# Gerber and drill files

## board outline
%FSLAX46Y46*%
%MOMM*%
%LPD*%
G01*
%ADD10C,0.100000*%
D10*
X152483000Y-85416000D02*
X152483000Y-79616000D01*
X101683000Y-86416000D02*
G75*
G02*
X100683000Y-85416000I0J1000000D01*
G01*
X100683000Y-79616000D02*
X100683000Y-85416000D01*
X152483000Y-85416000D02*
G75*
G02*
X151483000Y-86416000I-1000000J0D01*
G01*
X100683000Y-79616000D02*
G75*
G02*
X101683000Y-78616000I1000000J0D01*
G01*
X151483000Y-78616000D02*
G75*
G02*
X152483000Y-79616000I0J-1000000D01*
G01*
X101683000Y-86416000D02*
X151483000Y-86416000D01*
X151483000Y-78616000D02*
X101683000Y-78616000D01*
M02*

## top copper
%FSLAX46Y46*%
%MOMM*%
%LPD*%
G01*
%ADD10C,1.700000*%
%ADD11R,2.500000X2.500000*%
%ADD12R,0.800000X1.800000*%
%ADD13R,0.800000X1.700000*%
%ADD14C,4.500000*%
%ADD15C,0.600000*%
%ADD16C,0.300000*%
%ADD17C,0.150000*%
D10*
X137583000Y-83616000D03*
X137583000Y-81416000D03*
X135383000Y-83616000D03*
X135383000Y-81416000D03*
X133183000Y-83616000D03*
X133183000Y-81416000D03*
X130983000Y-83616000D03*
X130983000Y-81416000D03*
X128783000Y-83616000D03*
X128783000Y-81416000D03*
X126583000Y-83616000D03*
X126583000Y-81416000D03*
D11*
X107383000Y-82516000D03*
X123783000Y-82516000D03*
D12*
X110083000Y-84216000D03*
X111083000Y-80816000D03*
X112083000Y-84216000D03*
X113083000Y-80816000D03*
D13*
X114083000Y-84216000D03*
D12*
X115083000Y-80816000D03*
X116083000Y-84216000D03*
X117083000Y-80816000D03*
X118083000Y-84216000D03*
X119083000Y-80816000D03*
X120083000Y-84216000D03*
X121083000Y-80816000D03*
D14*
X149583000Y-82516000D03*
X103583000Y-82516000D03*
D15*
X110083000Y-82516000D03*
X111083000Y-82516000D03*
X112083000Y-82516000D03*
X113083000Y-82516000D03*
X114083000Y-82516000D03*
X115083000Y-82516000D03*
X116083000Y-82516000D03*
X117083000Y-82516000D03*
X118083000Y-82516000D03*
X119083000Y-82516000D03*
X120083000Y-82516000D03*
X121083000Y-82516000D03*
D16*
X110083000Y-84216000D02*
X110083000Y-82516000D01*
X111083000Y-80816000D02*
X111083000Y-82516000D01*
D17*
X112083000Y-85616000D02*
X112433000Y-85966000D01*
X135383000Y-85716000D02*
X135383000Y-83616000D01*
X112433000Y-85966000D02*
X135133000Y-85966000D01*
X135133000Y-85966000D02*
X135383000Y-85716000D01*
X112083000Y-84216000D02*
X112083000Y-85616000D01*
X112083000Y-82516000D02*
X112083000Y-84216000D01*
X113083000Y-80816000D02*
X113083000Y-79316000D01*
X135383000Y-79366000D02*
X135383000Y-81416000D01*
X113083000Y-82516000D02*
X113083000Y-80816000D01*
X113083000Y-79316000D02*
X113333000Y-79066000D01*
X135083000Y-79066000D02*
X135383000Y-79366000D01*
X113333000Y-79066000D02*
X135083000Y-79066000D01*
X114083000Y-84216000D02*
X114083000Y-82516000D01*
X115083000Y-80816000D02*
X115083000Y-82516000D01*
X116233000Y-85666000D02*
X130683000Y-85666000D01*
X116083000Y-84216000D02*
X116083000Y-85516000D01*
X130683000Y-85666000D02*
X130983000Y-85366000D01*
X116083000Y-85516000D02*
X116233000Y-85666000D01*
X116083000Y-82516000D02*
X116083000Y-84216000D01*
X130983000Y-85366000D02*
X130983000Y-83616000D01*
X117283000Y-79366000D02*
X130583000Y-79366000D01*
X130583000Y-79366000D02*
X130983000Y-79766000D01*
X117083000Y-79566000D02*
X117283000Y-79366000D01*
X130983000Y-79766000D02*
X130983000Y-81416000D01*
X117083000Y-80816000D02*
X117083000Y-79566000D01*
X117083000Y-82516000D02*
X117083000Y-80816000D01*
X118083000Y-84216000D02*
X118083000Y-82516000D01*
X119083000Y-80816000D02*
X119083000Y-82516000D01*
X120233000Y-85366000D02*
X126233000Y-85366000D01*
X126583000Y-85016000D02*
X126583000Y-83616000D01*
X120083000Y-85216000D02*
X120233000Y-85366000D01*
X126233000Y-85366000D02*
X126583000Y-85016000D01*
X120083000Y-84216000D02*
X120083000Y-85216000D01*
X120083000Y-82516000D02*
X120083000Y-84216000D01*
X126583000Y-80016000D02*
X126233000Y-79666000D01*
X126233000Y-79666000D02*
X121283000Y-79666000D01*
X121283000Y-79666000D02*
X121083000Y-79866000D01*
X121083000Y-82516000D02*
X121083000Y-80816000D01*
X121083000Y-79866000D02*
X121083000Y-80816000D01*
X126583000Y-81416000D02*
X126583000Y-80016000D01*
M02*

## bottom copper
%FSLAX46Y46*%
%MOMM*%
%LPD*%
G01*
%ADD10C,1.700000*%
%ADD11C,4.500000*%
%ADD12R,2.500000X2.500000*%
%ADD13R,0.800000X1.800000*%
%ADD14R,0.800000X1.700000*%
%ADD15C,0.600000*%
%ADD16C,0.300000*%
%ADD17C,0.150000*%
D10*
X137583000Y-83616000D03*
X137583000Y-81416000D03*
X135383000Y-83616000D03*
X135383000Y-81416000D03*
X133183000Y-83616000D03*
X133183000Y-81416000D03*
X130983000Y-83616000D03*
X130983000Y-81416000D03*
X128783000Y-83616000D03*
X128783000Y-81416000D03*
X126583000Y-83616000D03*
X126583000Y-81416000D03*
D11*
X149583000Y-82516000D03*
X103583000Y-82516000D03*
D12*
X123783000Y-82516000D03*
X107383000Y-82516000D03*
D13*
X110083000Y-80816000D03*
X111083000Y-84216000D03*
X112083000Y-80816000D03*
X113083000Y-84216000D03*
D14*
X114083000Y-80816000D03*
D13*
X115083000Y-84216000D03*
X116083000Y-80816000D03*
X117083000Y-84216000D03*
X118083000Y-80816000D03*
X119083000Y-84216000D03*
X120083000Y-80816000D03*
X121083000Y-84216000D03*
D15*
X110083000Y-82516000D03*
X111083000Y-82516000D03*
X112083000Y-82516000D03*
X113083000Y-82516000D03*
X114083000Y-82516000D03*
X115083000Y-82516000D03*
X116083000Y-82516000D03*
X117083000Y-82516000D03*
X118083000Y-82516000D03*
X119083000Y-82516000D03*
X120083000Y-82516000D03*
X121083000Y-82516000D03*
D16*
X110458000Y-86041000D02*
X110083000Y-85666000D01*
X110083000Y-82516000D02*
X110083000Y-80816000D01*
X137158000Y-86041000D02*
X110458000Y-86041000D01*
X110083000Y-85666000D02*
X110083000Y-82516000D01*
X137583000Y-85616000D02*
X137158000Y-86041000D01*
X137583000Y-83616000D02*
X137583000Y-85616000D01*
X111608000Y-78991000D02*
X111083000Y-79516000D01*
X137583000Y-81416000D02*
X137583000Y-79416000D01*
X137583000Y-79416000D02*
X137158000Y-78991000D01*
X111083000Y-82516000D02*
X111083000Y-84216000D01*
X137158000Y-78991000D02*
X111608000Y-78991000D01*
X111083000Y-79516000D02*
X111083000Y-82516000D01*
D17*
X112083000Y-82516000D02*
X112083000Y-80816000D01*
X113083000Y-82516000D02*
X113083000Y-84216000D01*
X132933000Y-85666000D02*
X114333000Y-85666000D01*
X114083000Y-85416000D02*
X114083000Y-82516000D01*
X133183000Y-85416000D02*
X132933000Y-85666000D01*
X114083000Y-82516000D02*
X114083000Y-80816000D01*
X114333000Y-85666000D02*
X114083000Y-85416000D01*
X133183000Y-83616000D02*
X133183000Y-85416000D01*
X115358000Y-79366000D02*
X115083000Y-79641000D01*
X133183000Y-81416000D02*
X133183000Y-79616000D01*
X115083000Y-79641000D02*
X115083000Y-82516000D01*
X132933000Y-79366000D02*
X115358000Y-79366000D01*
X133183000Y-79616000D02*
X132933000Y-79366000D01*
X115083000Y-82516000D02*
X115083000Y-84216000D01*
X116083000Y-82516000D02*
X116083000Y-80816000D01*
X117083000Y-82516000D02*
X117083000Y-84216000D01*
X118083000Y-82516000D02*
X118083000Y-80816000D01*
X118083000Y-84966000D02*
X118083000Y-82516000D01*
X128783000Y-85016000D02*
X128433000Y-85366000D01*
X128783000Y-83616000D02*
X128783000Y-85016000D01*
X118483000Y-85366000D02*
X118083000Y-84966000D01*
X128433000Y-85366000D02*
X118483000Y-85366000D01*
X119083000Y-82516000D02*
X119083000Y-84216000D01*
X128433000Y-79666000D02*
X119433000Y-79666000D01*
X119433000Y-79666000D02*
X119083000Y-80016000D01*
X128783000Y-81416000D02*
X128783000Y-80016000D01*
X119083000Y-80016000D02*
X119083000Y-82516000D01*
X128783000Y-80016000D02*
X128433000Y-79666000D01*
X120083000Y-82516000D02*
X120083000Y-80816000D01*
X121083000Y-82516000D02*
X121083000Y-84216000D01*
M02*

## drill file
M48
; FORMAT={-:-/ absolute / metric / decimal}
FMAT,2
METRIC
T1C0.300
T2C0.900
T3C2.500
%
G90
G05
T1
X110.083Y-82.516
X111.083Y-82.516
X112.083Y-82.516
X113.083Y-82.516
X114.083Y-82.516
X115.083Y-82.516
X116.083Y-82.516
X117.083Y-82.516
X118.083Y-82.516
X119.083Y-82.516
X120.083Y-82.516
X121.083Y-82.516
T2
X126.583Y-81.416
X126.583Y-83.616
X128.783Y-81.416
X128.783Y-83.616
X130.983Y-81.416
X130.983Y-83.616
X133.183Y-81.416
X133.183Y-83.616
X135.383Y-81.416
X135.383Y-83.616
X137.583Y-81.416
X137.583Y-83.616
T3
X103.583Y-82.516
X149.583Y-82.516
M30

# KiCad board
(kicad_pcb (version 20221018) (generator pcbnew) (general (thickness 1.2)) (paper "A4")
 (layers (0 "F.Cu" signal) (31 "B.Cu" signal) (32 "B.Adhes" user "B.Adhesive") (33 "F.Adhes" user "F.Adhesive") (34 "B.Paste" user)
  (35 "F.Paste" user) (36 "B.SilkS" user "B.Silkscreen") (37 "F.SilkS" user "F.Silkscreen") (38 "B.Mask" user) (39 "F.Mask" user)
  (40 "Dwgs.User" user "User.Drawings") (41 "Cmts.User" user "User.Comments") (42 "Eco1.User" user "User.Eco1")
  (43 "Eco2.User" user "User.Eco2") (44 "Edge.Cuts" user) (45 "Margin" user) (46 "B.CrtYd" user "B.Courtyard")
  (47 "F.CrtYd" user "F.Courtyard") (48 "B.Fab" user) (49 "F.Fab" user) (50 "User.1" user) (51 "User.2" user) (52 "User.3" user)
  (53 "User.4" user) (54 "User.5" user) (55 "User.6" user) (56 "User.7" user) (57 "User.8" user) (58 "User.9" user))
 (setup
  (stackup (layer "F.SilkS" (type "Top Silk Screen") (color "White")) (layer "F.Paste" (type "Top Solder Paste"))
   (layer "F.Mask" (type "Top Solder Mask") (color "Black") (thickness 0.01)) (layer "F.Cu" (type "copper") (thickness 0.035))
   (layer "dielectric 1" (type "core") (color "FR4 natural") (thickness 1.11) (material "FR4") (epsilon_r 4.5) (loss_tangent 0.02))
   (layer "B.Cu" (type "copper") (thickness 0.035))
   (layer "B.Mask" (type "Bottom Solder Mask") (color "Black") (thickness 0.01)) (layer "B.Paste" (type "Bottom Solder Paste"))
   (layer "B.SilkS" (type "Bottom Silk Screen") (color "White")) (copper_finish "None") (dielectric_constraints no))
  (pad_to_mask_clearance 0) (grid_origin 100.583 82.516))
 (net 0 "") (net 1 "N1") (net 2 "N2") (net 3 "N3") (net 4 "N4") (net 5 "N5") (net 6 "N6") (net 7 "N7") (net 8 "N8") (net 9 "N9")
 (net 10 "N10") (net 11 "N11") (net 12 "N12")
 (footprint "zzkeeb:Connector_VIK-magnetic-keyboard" (layer "F.Cu") (at 132.083 82.516 90)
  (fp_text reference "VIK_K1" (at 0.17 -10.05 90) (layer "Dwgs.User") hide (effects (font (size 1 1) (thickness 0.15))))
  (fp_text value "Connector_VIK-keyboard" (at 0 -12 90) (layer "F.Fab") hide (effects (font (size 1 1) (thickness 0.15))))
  (pad "1" thru_hole circle (at -1.1 5.5 270) (size 1.7 1.7) (drill 0.9) (layers "*.Cu" "*.Mask") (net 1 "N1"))
  (pad "2" thru_hole circle (at 1.1 5.5 270) (size 1.7 1.7) (drill 0.9) (layers "*.Cu" "*.Mask") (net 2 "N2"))
  (pad "3" thru_hole circle (at -1.1 3.3 270) (size 1.7 1.7) (drill 0.9) (layers "*.Cu" "*.Mask") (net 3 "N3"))
  (pad "4" thru_hole circle (at 1.1 3.3 270) (size 1.7 1.7) (drill 0.9) (layers "*.Cu" "*.Mask") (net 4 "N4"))
  (pad "5" thru_hole circle (at -1.1 1.1 270) (size 1.7 1.7) (drill 0.9) (layers "*.Cu" "*.Mask") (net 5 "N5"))
  (pad "6" thru_hole circle (at 1.1 1.1 270) (size 1.7 1.7) (drill 0.9) (layers "*.Cu" "*.Mask") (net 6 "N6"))
  (pad "7" thru_hole circle (at -1.1 -1.1 270) (size 1.7 1.7) (drill 0.9) (layers "*.Cu" "*.Mask") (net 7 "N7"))
  (pad "8" thru_hole circle (at 1.1 -1.1 270) (size 1.7 1.7) (drill 0.9) (layers "*.Cu" "*.Mask") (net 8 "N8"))
  (pad "9" thru_hole circle (at -1.1 -3.3 270) (size 1.7 1.7) (drill 0.9) (layers "*.Cu" "*.Mask") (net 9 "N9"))
  (pad "10" thru_hole circle (at 1.1 -3.3 270) (size 1.7 1.7) (drill 0.9) (layers "*.Cu" "*.Mask") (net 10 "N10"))
  (pad "11" thru_hole circle (at -1.1 -5.5 270) (size 1.7 1.7) (drill 0.9) (layers "*.Cu" "*.Mask") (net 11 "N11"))
  (pad "12" thru_hole circle (at 1.1 -5.5 270) (size 1.7 1.7) (drill 0.9) (layers "*.Cu" "*.Mask") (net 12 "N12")))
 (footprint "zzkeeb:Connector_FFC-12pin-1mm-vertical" (layer "F.Cu") (at 115.583 82.516 90)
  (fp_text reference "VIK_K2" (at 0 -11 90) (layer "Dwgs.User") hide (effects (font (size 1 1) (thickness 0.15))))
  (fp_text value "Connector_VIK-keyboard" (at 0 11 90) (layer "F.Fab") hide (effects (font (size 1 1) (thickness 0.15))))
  (pad "" smd rect (at 0 -8.2 90) (size 2.5 2.5) (layers "F.Cu" "F.Paste" "F.Mask"))
  (pad "" smd rect (at 0 8.2 90) (size 2.5 2.5) (layers "F.Cu" "F.Paste" "F.Mask"))
  (pad "1" smd rect (at -1.7 -5.5 90) (size 1.8 0.8) (layers "F.Cu" "F.Paste" "F.Mask") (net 1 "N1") (thermal_bridge_angle 45))
  (pad "2" smd rect (at 1.7 -4.5 90) (size 1.8 0.8) (layers "F.Cu" "F.Paste" "F.Mask") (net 2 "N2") (thermal_bridge_angle 45))
  (pad "3" smd rect (at -1.7 -3.5 90) (size 1.8 0.8) (layers "F.Cu" "F.Paste" "F.Mask") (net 3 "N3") (thermal_bridge_angle 45))
  (pad "4" smd rect (at 1.7 -2.5 90) (size 1.8 0.8) (layers "F.Cu" "F.Paste" "F.Mask") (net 4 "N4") (thermal_bridge_angle 45))
  (pad "5" smd rect (at -1.7 -1.5 90) (size 1.7 0.8) (layers "F.Cu" "F.Paste" "F.Mask") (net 5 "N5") (thermal_bridge_angle 45))
  (pad "6" smd rect (at 1.7 -0.5 90) (size 1.8 0.8) (layers "F.Cu" "F.Paste" "F.Mask") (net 6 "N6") (thermal_bridge_angle 45))
  (pad "7" smd rect (at -1.7 0.5 90) (size 1.8 0.8) (layers "F.Cu" "F.Paste" "F.Mask") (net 7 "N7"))
  (pad "8" smd rect (at 1.7 1.5 90) (size 1.8 0.8) (layers "F.Cu" "F.Paste" "F.Mask") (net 8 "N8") (thermal_bridge_angle 45))
  (pad "9" smd rect (at -1.7 2.5 90) (size 1.8 0.8) (layers "F.Cu" "F.Paste" "F.Mask") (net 9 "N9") (thermal_bridge_angle 45))
  (pad "10" smd rect (at 1.7 3.5 90) (size 1.8 0.8) (layers "F.Cu" "F.Paste" "F.Mask") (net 10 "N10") (thermal_bridge_angle 45))
  (pad "11" smd rect (at -1.7 4.5 90) (size 1.8 0.8) (layers "F.Cu" "F.Paste" "F.Mask") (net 11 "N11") (thermal_bridge_angle 45))
  (pad "12" smd rect (at 1.7 5.5 90) (size 1.8 0.8) (layers "F.Cu" "F.Paste" "F.Mask") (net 12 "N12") (thermal_bridge_angle 45)))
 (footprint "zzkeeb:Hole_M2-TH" (layer "F.Cu") (at 149.583 82.516)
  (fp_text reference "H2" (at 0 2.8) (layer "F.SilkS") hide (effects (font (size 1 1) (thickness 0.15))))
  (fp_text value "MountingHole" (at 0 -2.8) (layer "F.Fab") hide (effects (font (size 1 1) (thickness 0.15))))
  (pad "" thru_hole circle (at 0 0) (size 4.5 4.5) (drill 2.5) (layers "*.Cu" "*.Mask")))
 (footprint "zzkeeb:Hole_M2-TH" (layer "B.Cu") (at 103.583 82.516 180)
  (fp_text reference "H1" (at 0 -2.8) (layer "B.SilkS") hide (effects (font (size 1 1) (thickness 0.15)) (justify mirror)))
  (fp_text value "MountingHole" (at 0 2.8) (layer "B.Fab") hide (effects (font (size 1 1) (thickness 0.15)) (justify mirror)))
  (pad "" thru_hole circle (at 0 0 180) (size 4.5 4.5) (drill 2.5) (layers "*.Cu" "*.Mask")))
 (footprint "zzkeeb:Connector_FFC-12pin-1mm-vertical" (layer "B.Cu") (at 115.583 82.516 -90)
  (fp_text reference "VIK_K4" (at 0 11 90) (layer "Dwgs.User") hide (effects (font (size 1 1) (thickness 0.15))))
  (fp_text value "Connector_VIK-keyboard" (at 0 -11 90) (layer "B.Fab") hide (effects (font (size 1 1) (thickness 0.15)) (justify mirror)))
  (pad "" smd rect (at 0 -8.2 270) (size 2.5 2.5) (layers "B.Cu" "B.Paste" "B.Mask"))
  (pad "" smd rect (at 0 8.2 270) (size 2.5 2.5) (layers "B.Cu" "B.Paste" "B.Mask"))
  (pad "1" smd rect (at -1.7 5.5 270) (size 1.8 0.8) (layers "B.Cu" "B.Paste" "B.Mask") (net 1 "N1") (thermal_bridge_angle 45))
  (pad "2" smd rect (at 1.7 4.5 270) (size 1.8 0.8) (layers "B.Cu" "B.Paste" "B.Mask") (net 2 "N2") (thermal_bridge_angle 45))
  (pad "3" smd rect (at -1.7 3.5 270) (size 1.8 0.8) (layers "B.Cu" "B.Paste" "B.Mask") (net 3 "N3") (thermal_bridge_angle 45))
  (pad "4" smd rect (at 1.7 2.5 270) (size 1.8 0.8) (layers "B.Cu" "B.Paste" "B.Mask") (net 4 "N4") (thermal_bridge_angle 45))
  (pad "5" smd rect (at -1.7 1.5 270) (size 1.7 0.8) (layers "B.Cu" "B.Paste" "B.Mask") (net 5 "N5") (thermal_bridge_angle 45))
  (pad "6" smd rect (at 1.7 0.5 270) (size 1.8 0.8) (layers "B.Cu" "B.Paste" "B.Mask") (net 6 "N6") (thermal_bridge_angle 45))
  (pad "7" smd rect (at -1.7 -0.5 270) (size 1.8 0.8) (layers "B.Cu" "B.Paste" "B.Mask") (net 7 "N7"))
  (pad "8" smd rect (at 1.7 -1.5 270) (size 1.8 0.8) (layers "B.Cu" "B.Paste" "B.Mask") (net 8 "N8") (thermal_bridge_angle 45))
  (pad "9" smd rect (at -1.7 -2.5 270) (size 1.8 0.8) (layers "B.Cu" "B.Paste" "B.Mask") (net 9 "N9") (thermal_bridge_angle 45))
  (pad "10" smd rect (at 1.7 -3.5 270) (size 1.8 0.8) (layers "B.Cu" "B.Paste" "B.Mask") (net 10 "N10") (thermal_bridge_angle 45))
  (pad "11" smd rect (at -1.7 -4.5 270) (size 1.8 0.8) (layers "B.Cu" "B.Paste" "B.Mask") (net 11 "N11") (thermal_bridge_angle 45))
  (pad "12" smd rect (at 1.7 -5.5 270) (size 1.8 0.8) (layers "B.Cu" "B.Paste" "B.Mask") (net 12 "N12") (thermal_bridge_angle 45)))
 (gr_line (start 152.483 85.416) (end 152.483 79.616) (stroke (width 0.1) (type default)) (layer "Edge.Cuts"))
 (gr_arc (start 101.683 86.416) (mid 100.975893 86.123107) (end 100.683 85.416) (stroke (width 0.1) (type default)) (layer "Edge.Cuts"))
 (gr_line (start 100.683 79.616) (end 100.683 85.416) (stroke (width 0.1) (type default)) (layer "Edge.Cuts"))
 (gr_arc (start 152.483 85.416) (mid 152.190107 86.123107) (end 151.483 86.416) (stroke (width 0.1) (type default)) (layer "Edge.Cuts"))
 (gr_arc (start 100.683 79.616) (mid 100.975893 78.908893) (end 101.683 78.616) (stroke (width 0.1) (type default)) (layer "Edge.Cuts"))
 (gr_arc (start 151.483 78.616) (mid 152.190107 78.908893) (end 152.483 79.616) (stroke (width 0.1) (type default)) (layer "Edge.Cuts"))
 (gr_line (start 101.683 86.416) (end 151.483 86.416) (stroke (width 0.1) (type default)) (layer "Edge.Cuts"))
 (gr_line (start 151.483 78.616) (end 101.683 78.616) (stroke (width 0.1) (type default)) (layer "Edge.Cuts"))
 (segment (start 110.083 84.216) (end 110.083 82.516) (width 0.3) (layer "F.Cu") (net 1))
 (via (at 110.083 82.516) (size 0.6) (drill 0.3) (layers "F.Cu" "B.Cu") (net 1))
 (segment (start 110.458 86.041) (end 110.083 85.666) (width 0.3) (layer "B.Cu") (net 1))
 (segment (start 110.083 82.516) (end 110.083 80.816) (width 0.3) (layer "B.Cu") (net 1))
 (segment (start 137.158 86.041) (end 110.458 86.041) (width 0.3) (layer "B.Cu") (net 1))
 (segment (start 110.083 85.666) (end 110.083 82.516) (width 0.3) (layer "B.Cu") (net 1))
 (segment (start 137.583 85.616) (end 137.158 86.041) (width 0.3) (layer "B.Cu") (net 1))
 (segment (start 137.583 83.616) (end 137.583 85.616) (width 0.3) (layer "B.Cu") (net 1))
 (segment (start 111.083 80.816) (end 111.083 82.516) (width 0.3) (layer "F.Cu") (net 2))
 (via (at 111.083 82.516) (size 0.6) (drill 0.3) (layers "F.Cu" "B.Cu") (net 2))
 (segment (start 111.608 78.991) (end 111.083 79.516) (width 0.3) (layer "B.Cu") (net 2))
 (segment (start 137.583 81.416) (end 137.583 79.416) (width 0.3) (layer "B.Cu") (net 2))
 (segment (start 137.583 79.416) (end 137.158 78.991) (width 0.3) (layer "B.Cu") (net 2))
 (segment (start 111.083 82.516) (end 111.083 84.216) (width 0.3) (layer "B.Cu") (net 2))
 (segment (start 137.158 78.991) (end 111.608 78.991) (width 0.3) (layer "B.Cu") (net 2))
 (segment (start 111.083 79.516) (end 111.083 82.516) (width 0.3) (layer "B.Cu") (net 2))
 (segment (start 112.083 85.616) (end 112.433 85.966) (width 0.15) (layer "F.Cu") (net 3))
 (segment (start 135.383 85.716) (end 135.383 83.616) (width 0.15) (layer "F.Cu") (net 3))
 (segment (start 112.433 85.966) (end 135.133 85.966) (width 0.15) (layer "F.Cu") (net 3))
 (segment (start 135.133 85.966) (end 135.383 85.716) (width 0.15) (layer "F.Cu") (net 3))
 (segment (start 112.083 84.216) (end 112.083 85.616) (width 0.15) (layer "F.Cu") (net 3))
 (segment (start 112.083 82.516) (end 112.083 84.216) (width 0.15) (layer "F.Cu") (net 3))
 (via (at 112.083 82.516) (size 0.6) (drill 0.3) (layers "F.Cu" "B.Cu") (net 3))
 (segment (start 112.083 82.516) (end 112.083 80.816) (width 0.15) (layer "B.Cu") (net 3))
 (segment (start 113.083 80.816) (end 113.083 79.316) (width 0.15) (layer "F.Cu") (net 4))
 (segment (start 135.383 79.366) (end 135.383 81.416) (width 0.15) (layer "F.Cu") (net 4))
 (segment (start 113.083 82.516) (end 113.083 80.816) (width 0.15) (layer "F.Cu") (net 4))
 (segment (start 113.083 79.316) (end 113.333 79.066) (width 0.15) (layer "F.Cu") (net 4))
 (segment (start 135.083 79.066) (end 135.383 79.366) (width 0.15) (layer "F.Cu") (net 4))
 (segment (start 113.333 79.066) (end 135.083 79.066) (width 0.15) (layer "F.Cu") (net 4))
 (via (at 113.083 82.516) (size 0.6) (drill 0.3) (layers "F.Cu" "B.Cu") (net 4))
 (segment (start 113.083 82.516) (end 113.083 84.216) (width 0.15) (layer "B.Cu") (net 4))
 (segment (start 114.083 84.216) (end 114.083 82.516) (width 0.15) (layer "F.Cu") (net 5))
 (via (at 114.083 82.516) (size 0.6) (drill 0.3) (layers "F.Cu" "B.Cu") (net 5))
 (segment (start 132.933 85.666) (end 114.333 85.666) (width 0.15) (layer "B.Cu") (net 5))
 (segment (start 114.083 85.416) (end 114.083 82.516) (width 0.15) (layer "B.Cu") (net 5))
 (segment (start 133.183 85.416) (end 132.933 85.666) (width 0.15) (layer "B.Cu") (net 5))
 (segment (start 114.083 82.516) (end 114.083 80.816) (width 0.15) (layer "B.Cu") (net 5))
 (segment (start 114.333 85.666) (end 114.083 85.416) (width 0.15) (layer "B.Cu") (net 5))
 (segment (start 133.183 83.616) (end 133.183 85.416) (width 0.15) (layer "B.Cu") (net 5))
 (segment (start 115.083 80.816) (end 115.083 82.516) (width 0.15) (layer "F.Cu") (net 6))
 (via (at 115.083 82.516) (size 0.6) (drill 0.3) (layers "F.Cu" "B.Cu") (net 6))
 (segment (start 115.358 79.366) (end 115.083 79.641) (width 0.15) (layer "B.Cu") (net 6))
 (segment (start 133.183 81.416) (end 133.183 79.616) (width 0.15) (layer "B.Cu") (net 6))
 (segment (start 115.083 79.641) (end 115.083 82.516) (width 0.15) (layer "B.Cu") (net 6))
 (segment (start 132.933 79.366) (end 115.358 79.366) (width 0.15) (layer "B.Cu") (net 6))
 (segment (start 133.183 79.616) (end 132.933 79.366) (width 0.15) (layer "B.Cu") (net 6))
 (segment (start 115.083 82.516) (end 115.083 84.216) (width 0.15) (layer "B.Cu") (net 6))
 (segment (start 116.233 85.666) (end 130.683 85.666) (width 0.15) (layer "F.Cu") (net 7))
 (segment (start 116.083 84.216) (end 116.083 85.516) (width 0.15) (layer "F.Cu") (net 7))
 (segment (start 130.683 85.666) (end 130.983 85.366) (width 0.15) (layer "F.Cu") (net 7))
 (segment (start 116.083 85.516) (end 116.233 85.666) (width 0.15) (layer "F.Cu") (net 7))
 (segment (start 116.083 82.516) (end 116.083 84.216) (width 0.15) (layer "F.Cu") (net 7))
 (segment (start 130.983 85.366) (end 130.983 83.616) (width 0.15) (layer "F.Cu") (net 7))
 (via (at 116.083 82.516) (size 0.6) (drill 0.3) (layers "F.Cu" "B.Cu") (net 7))
 (segment (start 116.083 82.516) (end 116.083 80.816) (width 0.15) (layer "B.Cu") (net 7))
 (segment (start 117.283 79.366) (end 130.583 79.366) (width 0.15) (layer "F.Cu") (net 8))
 (segment (start 130.583 79.366) (end 130.983 79.766) (width 0.15) (layer "F.Cu") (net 8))
 (segment (start 117.083 79.566) (end 117.283 79.366) (width 0.15) (layer "F.Cu") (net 8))
 (segment (start 130.983 79.766) (end 130.983 81.416) (width 0.15) (layer "F.Cu") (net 8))
 (segment (start 117.083 80.816) (end 117.083 79.566) (width 0.15) (layer "F.Cu") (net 8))
 (segment (start 117.083 82.516) (end 117.083 80.816) (width 0.15) (layer "F.Cu") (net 8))
 (via (at 117.083 82.516) (size 0.6) (drill 0.3) (layers "F.Cu" "B.Cu") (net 8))
 (segment (start 117.083 82.516) (end 117.083 84.216) (width 0.15) (layer "B.Cu") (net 8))
 (segment (start 118.083 84.216) (end 118.083 82.516) (width 0.15) (layer "F.Cu") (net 9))
 (via (at 118.083 82.516) (size 0.6) (drill 0.3) (layers "F.Cu" "B.Cu") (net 9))
 (segment (start 118.083 82.516) (end 118.083 80.816) (width 0.15) (layer "B.Cu") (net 9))
 (segment (start 118.083 84.966) (end 118.083 82.516) (width 0.15) (layer "B.Cu") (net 9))
 (segment (start 128.783 85.016) (end 128.433 85.366) (width 0.15) (layer "B.Cu") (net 9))
 (segment (start 128.783 83.616) (end 128.783 85.016) (width 0.15) (layer "B.Cu") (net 9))
 (segment (start 118.483 85.366) (end 118.083 84.966) (width 0.15) (layer "B.Cu") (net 9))
 (segment (start 128.433 85.366) (end 118.483 85.366) (width 0.15) (layer "B.Cu") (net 9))
 (segment (start 119.083 80.816) (end 119.083 82.516) (width 0.15) (layer "F.Cu") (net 10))
 (via (at 119.083 82.516) (size 0.6) (drill 0.3) (layers "F.Cu" "B.Cu") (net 10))
 (segment (start 119.083 82.516) (end 119.083 84.216) (width 0.15) (layer "B.Cu") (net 10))
 (segment (start 128.433 79.666) (end 119.433 79.666) (width 0.15) (layer "B.Cu") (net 10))
 (segment (start 119.433 79.666) (end 119.083 80.016) (width 0.15) (layer "B.Cu") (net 10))
 (segment (start 128.783 81.416) (end 128.783 80.016) (width 0.15) (layer "B.Cu") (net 10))
 (segment (start 119.083 80.016) (end 119.083 82.516) (width 0.15) (layer "B.Cu") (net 10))
 (segment (start 128.783 80.016) (end 128.433 79.666) (width 0.15) (layer "B.Cu") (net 10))
 (segment (start 120.233 85.366) (end 126.233 85.366) (width 0.15) (layer "F.Cu") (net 11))
 (segment (start 126.583 85.016) (end 126.583 83.616) (width 0.15) (layer "F.Cu") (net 11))
 (segment (start 120.083 85.216) (end 120.233 85.366) (width 0.15) (layer "F.Cu") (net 11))
 (segment (start 126.233 85.366) (end 126.583 85.016) (width 0.15) (layer "F.Cu") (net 11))
 (segment (start 120.083 84.216) (end 120.083 85.216) (width 0.15) (layer "F.Cu") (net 11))
 (segment (start 120.083 82.516) (end 120.083 84.216) (width 0.15) (layer "F.Cu") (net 11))
 (via (at 120.083 82.516) (size 0.6) (drill 0.3) (layers "F.Cu" "B.Cu") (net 11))
 (segment (start 120.083 82.516) (end 120.083 80.816) (width 0.15) (layer "B.Cu") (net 11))
 (segment (start 126.583 80.016) (end 126.233 79.666) (width 0.15) (layer "F.Cu") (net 12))
 (segment (start 126.233 79.666) (end 121.283 79.666) (width 0.15) (layer "F.Cu") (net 12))
 (segment (start 121.283 79.666) (end 121.083 79.866) (width 0.15) (layer "F.Cu") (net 12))
 (segment (start 121.083 82.516) (end 121.083 80.816) (width 0.15) (layer "F.Cu") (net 12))
 (segment (start 121.083 79.866) (end 121.083 80.816) (width 0.15) (layer "F.Cu") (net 12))
 (segment (start 126.583 81.416) (end 126.583 80.016) (width 0.15) (layer "F.Cu") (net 12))
 (via (at 121.083 82.516) (size 0.6) (drill 0.3) (layers "F.Cu" "B.Cu") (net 12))
 (segment (start 121.083 82.516) (end 121.083 84.216) (width 0.15) (layer "B.Cu") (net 12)))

